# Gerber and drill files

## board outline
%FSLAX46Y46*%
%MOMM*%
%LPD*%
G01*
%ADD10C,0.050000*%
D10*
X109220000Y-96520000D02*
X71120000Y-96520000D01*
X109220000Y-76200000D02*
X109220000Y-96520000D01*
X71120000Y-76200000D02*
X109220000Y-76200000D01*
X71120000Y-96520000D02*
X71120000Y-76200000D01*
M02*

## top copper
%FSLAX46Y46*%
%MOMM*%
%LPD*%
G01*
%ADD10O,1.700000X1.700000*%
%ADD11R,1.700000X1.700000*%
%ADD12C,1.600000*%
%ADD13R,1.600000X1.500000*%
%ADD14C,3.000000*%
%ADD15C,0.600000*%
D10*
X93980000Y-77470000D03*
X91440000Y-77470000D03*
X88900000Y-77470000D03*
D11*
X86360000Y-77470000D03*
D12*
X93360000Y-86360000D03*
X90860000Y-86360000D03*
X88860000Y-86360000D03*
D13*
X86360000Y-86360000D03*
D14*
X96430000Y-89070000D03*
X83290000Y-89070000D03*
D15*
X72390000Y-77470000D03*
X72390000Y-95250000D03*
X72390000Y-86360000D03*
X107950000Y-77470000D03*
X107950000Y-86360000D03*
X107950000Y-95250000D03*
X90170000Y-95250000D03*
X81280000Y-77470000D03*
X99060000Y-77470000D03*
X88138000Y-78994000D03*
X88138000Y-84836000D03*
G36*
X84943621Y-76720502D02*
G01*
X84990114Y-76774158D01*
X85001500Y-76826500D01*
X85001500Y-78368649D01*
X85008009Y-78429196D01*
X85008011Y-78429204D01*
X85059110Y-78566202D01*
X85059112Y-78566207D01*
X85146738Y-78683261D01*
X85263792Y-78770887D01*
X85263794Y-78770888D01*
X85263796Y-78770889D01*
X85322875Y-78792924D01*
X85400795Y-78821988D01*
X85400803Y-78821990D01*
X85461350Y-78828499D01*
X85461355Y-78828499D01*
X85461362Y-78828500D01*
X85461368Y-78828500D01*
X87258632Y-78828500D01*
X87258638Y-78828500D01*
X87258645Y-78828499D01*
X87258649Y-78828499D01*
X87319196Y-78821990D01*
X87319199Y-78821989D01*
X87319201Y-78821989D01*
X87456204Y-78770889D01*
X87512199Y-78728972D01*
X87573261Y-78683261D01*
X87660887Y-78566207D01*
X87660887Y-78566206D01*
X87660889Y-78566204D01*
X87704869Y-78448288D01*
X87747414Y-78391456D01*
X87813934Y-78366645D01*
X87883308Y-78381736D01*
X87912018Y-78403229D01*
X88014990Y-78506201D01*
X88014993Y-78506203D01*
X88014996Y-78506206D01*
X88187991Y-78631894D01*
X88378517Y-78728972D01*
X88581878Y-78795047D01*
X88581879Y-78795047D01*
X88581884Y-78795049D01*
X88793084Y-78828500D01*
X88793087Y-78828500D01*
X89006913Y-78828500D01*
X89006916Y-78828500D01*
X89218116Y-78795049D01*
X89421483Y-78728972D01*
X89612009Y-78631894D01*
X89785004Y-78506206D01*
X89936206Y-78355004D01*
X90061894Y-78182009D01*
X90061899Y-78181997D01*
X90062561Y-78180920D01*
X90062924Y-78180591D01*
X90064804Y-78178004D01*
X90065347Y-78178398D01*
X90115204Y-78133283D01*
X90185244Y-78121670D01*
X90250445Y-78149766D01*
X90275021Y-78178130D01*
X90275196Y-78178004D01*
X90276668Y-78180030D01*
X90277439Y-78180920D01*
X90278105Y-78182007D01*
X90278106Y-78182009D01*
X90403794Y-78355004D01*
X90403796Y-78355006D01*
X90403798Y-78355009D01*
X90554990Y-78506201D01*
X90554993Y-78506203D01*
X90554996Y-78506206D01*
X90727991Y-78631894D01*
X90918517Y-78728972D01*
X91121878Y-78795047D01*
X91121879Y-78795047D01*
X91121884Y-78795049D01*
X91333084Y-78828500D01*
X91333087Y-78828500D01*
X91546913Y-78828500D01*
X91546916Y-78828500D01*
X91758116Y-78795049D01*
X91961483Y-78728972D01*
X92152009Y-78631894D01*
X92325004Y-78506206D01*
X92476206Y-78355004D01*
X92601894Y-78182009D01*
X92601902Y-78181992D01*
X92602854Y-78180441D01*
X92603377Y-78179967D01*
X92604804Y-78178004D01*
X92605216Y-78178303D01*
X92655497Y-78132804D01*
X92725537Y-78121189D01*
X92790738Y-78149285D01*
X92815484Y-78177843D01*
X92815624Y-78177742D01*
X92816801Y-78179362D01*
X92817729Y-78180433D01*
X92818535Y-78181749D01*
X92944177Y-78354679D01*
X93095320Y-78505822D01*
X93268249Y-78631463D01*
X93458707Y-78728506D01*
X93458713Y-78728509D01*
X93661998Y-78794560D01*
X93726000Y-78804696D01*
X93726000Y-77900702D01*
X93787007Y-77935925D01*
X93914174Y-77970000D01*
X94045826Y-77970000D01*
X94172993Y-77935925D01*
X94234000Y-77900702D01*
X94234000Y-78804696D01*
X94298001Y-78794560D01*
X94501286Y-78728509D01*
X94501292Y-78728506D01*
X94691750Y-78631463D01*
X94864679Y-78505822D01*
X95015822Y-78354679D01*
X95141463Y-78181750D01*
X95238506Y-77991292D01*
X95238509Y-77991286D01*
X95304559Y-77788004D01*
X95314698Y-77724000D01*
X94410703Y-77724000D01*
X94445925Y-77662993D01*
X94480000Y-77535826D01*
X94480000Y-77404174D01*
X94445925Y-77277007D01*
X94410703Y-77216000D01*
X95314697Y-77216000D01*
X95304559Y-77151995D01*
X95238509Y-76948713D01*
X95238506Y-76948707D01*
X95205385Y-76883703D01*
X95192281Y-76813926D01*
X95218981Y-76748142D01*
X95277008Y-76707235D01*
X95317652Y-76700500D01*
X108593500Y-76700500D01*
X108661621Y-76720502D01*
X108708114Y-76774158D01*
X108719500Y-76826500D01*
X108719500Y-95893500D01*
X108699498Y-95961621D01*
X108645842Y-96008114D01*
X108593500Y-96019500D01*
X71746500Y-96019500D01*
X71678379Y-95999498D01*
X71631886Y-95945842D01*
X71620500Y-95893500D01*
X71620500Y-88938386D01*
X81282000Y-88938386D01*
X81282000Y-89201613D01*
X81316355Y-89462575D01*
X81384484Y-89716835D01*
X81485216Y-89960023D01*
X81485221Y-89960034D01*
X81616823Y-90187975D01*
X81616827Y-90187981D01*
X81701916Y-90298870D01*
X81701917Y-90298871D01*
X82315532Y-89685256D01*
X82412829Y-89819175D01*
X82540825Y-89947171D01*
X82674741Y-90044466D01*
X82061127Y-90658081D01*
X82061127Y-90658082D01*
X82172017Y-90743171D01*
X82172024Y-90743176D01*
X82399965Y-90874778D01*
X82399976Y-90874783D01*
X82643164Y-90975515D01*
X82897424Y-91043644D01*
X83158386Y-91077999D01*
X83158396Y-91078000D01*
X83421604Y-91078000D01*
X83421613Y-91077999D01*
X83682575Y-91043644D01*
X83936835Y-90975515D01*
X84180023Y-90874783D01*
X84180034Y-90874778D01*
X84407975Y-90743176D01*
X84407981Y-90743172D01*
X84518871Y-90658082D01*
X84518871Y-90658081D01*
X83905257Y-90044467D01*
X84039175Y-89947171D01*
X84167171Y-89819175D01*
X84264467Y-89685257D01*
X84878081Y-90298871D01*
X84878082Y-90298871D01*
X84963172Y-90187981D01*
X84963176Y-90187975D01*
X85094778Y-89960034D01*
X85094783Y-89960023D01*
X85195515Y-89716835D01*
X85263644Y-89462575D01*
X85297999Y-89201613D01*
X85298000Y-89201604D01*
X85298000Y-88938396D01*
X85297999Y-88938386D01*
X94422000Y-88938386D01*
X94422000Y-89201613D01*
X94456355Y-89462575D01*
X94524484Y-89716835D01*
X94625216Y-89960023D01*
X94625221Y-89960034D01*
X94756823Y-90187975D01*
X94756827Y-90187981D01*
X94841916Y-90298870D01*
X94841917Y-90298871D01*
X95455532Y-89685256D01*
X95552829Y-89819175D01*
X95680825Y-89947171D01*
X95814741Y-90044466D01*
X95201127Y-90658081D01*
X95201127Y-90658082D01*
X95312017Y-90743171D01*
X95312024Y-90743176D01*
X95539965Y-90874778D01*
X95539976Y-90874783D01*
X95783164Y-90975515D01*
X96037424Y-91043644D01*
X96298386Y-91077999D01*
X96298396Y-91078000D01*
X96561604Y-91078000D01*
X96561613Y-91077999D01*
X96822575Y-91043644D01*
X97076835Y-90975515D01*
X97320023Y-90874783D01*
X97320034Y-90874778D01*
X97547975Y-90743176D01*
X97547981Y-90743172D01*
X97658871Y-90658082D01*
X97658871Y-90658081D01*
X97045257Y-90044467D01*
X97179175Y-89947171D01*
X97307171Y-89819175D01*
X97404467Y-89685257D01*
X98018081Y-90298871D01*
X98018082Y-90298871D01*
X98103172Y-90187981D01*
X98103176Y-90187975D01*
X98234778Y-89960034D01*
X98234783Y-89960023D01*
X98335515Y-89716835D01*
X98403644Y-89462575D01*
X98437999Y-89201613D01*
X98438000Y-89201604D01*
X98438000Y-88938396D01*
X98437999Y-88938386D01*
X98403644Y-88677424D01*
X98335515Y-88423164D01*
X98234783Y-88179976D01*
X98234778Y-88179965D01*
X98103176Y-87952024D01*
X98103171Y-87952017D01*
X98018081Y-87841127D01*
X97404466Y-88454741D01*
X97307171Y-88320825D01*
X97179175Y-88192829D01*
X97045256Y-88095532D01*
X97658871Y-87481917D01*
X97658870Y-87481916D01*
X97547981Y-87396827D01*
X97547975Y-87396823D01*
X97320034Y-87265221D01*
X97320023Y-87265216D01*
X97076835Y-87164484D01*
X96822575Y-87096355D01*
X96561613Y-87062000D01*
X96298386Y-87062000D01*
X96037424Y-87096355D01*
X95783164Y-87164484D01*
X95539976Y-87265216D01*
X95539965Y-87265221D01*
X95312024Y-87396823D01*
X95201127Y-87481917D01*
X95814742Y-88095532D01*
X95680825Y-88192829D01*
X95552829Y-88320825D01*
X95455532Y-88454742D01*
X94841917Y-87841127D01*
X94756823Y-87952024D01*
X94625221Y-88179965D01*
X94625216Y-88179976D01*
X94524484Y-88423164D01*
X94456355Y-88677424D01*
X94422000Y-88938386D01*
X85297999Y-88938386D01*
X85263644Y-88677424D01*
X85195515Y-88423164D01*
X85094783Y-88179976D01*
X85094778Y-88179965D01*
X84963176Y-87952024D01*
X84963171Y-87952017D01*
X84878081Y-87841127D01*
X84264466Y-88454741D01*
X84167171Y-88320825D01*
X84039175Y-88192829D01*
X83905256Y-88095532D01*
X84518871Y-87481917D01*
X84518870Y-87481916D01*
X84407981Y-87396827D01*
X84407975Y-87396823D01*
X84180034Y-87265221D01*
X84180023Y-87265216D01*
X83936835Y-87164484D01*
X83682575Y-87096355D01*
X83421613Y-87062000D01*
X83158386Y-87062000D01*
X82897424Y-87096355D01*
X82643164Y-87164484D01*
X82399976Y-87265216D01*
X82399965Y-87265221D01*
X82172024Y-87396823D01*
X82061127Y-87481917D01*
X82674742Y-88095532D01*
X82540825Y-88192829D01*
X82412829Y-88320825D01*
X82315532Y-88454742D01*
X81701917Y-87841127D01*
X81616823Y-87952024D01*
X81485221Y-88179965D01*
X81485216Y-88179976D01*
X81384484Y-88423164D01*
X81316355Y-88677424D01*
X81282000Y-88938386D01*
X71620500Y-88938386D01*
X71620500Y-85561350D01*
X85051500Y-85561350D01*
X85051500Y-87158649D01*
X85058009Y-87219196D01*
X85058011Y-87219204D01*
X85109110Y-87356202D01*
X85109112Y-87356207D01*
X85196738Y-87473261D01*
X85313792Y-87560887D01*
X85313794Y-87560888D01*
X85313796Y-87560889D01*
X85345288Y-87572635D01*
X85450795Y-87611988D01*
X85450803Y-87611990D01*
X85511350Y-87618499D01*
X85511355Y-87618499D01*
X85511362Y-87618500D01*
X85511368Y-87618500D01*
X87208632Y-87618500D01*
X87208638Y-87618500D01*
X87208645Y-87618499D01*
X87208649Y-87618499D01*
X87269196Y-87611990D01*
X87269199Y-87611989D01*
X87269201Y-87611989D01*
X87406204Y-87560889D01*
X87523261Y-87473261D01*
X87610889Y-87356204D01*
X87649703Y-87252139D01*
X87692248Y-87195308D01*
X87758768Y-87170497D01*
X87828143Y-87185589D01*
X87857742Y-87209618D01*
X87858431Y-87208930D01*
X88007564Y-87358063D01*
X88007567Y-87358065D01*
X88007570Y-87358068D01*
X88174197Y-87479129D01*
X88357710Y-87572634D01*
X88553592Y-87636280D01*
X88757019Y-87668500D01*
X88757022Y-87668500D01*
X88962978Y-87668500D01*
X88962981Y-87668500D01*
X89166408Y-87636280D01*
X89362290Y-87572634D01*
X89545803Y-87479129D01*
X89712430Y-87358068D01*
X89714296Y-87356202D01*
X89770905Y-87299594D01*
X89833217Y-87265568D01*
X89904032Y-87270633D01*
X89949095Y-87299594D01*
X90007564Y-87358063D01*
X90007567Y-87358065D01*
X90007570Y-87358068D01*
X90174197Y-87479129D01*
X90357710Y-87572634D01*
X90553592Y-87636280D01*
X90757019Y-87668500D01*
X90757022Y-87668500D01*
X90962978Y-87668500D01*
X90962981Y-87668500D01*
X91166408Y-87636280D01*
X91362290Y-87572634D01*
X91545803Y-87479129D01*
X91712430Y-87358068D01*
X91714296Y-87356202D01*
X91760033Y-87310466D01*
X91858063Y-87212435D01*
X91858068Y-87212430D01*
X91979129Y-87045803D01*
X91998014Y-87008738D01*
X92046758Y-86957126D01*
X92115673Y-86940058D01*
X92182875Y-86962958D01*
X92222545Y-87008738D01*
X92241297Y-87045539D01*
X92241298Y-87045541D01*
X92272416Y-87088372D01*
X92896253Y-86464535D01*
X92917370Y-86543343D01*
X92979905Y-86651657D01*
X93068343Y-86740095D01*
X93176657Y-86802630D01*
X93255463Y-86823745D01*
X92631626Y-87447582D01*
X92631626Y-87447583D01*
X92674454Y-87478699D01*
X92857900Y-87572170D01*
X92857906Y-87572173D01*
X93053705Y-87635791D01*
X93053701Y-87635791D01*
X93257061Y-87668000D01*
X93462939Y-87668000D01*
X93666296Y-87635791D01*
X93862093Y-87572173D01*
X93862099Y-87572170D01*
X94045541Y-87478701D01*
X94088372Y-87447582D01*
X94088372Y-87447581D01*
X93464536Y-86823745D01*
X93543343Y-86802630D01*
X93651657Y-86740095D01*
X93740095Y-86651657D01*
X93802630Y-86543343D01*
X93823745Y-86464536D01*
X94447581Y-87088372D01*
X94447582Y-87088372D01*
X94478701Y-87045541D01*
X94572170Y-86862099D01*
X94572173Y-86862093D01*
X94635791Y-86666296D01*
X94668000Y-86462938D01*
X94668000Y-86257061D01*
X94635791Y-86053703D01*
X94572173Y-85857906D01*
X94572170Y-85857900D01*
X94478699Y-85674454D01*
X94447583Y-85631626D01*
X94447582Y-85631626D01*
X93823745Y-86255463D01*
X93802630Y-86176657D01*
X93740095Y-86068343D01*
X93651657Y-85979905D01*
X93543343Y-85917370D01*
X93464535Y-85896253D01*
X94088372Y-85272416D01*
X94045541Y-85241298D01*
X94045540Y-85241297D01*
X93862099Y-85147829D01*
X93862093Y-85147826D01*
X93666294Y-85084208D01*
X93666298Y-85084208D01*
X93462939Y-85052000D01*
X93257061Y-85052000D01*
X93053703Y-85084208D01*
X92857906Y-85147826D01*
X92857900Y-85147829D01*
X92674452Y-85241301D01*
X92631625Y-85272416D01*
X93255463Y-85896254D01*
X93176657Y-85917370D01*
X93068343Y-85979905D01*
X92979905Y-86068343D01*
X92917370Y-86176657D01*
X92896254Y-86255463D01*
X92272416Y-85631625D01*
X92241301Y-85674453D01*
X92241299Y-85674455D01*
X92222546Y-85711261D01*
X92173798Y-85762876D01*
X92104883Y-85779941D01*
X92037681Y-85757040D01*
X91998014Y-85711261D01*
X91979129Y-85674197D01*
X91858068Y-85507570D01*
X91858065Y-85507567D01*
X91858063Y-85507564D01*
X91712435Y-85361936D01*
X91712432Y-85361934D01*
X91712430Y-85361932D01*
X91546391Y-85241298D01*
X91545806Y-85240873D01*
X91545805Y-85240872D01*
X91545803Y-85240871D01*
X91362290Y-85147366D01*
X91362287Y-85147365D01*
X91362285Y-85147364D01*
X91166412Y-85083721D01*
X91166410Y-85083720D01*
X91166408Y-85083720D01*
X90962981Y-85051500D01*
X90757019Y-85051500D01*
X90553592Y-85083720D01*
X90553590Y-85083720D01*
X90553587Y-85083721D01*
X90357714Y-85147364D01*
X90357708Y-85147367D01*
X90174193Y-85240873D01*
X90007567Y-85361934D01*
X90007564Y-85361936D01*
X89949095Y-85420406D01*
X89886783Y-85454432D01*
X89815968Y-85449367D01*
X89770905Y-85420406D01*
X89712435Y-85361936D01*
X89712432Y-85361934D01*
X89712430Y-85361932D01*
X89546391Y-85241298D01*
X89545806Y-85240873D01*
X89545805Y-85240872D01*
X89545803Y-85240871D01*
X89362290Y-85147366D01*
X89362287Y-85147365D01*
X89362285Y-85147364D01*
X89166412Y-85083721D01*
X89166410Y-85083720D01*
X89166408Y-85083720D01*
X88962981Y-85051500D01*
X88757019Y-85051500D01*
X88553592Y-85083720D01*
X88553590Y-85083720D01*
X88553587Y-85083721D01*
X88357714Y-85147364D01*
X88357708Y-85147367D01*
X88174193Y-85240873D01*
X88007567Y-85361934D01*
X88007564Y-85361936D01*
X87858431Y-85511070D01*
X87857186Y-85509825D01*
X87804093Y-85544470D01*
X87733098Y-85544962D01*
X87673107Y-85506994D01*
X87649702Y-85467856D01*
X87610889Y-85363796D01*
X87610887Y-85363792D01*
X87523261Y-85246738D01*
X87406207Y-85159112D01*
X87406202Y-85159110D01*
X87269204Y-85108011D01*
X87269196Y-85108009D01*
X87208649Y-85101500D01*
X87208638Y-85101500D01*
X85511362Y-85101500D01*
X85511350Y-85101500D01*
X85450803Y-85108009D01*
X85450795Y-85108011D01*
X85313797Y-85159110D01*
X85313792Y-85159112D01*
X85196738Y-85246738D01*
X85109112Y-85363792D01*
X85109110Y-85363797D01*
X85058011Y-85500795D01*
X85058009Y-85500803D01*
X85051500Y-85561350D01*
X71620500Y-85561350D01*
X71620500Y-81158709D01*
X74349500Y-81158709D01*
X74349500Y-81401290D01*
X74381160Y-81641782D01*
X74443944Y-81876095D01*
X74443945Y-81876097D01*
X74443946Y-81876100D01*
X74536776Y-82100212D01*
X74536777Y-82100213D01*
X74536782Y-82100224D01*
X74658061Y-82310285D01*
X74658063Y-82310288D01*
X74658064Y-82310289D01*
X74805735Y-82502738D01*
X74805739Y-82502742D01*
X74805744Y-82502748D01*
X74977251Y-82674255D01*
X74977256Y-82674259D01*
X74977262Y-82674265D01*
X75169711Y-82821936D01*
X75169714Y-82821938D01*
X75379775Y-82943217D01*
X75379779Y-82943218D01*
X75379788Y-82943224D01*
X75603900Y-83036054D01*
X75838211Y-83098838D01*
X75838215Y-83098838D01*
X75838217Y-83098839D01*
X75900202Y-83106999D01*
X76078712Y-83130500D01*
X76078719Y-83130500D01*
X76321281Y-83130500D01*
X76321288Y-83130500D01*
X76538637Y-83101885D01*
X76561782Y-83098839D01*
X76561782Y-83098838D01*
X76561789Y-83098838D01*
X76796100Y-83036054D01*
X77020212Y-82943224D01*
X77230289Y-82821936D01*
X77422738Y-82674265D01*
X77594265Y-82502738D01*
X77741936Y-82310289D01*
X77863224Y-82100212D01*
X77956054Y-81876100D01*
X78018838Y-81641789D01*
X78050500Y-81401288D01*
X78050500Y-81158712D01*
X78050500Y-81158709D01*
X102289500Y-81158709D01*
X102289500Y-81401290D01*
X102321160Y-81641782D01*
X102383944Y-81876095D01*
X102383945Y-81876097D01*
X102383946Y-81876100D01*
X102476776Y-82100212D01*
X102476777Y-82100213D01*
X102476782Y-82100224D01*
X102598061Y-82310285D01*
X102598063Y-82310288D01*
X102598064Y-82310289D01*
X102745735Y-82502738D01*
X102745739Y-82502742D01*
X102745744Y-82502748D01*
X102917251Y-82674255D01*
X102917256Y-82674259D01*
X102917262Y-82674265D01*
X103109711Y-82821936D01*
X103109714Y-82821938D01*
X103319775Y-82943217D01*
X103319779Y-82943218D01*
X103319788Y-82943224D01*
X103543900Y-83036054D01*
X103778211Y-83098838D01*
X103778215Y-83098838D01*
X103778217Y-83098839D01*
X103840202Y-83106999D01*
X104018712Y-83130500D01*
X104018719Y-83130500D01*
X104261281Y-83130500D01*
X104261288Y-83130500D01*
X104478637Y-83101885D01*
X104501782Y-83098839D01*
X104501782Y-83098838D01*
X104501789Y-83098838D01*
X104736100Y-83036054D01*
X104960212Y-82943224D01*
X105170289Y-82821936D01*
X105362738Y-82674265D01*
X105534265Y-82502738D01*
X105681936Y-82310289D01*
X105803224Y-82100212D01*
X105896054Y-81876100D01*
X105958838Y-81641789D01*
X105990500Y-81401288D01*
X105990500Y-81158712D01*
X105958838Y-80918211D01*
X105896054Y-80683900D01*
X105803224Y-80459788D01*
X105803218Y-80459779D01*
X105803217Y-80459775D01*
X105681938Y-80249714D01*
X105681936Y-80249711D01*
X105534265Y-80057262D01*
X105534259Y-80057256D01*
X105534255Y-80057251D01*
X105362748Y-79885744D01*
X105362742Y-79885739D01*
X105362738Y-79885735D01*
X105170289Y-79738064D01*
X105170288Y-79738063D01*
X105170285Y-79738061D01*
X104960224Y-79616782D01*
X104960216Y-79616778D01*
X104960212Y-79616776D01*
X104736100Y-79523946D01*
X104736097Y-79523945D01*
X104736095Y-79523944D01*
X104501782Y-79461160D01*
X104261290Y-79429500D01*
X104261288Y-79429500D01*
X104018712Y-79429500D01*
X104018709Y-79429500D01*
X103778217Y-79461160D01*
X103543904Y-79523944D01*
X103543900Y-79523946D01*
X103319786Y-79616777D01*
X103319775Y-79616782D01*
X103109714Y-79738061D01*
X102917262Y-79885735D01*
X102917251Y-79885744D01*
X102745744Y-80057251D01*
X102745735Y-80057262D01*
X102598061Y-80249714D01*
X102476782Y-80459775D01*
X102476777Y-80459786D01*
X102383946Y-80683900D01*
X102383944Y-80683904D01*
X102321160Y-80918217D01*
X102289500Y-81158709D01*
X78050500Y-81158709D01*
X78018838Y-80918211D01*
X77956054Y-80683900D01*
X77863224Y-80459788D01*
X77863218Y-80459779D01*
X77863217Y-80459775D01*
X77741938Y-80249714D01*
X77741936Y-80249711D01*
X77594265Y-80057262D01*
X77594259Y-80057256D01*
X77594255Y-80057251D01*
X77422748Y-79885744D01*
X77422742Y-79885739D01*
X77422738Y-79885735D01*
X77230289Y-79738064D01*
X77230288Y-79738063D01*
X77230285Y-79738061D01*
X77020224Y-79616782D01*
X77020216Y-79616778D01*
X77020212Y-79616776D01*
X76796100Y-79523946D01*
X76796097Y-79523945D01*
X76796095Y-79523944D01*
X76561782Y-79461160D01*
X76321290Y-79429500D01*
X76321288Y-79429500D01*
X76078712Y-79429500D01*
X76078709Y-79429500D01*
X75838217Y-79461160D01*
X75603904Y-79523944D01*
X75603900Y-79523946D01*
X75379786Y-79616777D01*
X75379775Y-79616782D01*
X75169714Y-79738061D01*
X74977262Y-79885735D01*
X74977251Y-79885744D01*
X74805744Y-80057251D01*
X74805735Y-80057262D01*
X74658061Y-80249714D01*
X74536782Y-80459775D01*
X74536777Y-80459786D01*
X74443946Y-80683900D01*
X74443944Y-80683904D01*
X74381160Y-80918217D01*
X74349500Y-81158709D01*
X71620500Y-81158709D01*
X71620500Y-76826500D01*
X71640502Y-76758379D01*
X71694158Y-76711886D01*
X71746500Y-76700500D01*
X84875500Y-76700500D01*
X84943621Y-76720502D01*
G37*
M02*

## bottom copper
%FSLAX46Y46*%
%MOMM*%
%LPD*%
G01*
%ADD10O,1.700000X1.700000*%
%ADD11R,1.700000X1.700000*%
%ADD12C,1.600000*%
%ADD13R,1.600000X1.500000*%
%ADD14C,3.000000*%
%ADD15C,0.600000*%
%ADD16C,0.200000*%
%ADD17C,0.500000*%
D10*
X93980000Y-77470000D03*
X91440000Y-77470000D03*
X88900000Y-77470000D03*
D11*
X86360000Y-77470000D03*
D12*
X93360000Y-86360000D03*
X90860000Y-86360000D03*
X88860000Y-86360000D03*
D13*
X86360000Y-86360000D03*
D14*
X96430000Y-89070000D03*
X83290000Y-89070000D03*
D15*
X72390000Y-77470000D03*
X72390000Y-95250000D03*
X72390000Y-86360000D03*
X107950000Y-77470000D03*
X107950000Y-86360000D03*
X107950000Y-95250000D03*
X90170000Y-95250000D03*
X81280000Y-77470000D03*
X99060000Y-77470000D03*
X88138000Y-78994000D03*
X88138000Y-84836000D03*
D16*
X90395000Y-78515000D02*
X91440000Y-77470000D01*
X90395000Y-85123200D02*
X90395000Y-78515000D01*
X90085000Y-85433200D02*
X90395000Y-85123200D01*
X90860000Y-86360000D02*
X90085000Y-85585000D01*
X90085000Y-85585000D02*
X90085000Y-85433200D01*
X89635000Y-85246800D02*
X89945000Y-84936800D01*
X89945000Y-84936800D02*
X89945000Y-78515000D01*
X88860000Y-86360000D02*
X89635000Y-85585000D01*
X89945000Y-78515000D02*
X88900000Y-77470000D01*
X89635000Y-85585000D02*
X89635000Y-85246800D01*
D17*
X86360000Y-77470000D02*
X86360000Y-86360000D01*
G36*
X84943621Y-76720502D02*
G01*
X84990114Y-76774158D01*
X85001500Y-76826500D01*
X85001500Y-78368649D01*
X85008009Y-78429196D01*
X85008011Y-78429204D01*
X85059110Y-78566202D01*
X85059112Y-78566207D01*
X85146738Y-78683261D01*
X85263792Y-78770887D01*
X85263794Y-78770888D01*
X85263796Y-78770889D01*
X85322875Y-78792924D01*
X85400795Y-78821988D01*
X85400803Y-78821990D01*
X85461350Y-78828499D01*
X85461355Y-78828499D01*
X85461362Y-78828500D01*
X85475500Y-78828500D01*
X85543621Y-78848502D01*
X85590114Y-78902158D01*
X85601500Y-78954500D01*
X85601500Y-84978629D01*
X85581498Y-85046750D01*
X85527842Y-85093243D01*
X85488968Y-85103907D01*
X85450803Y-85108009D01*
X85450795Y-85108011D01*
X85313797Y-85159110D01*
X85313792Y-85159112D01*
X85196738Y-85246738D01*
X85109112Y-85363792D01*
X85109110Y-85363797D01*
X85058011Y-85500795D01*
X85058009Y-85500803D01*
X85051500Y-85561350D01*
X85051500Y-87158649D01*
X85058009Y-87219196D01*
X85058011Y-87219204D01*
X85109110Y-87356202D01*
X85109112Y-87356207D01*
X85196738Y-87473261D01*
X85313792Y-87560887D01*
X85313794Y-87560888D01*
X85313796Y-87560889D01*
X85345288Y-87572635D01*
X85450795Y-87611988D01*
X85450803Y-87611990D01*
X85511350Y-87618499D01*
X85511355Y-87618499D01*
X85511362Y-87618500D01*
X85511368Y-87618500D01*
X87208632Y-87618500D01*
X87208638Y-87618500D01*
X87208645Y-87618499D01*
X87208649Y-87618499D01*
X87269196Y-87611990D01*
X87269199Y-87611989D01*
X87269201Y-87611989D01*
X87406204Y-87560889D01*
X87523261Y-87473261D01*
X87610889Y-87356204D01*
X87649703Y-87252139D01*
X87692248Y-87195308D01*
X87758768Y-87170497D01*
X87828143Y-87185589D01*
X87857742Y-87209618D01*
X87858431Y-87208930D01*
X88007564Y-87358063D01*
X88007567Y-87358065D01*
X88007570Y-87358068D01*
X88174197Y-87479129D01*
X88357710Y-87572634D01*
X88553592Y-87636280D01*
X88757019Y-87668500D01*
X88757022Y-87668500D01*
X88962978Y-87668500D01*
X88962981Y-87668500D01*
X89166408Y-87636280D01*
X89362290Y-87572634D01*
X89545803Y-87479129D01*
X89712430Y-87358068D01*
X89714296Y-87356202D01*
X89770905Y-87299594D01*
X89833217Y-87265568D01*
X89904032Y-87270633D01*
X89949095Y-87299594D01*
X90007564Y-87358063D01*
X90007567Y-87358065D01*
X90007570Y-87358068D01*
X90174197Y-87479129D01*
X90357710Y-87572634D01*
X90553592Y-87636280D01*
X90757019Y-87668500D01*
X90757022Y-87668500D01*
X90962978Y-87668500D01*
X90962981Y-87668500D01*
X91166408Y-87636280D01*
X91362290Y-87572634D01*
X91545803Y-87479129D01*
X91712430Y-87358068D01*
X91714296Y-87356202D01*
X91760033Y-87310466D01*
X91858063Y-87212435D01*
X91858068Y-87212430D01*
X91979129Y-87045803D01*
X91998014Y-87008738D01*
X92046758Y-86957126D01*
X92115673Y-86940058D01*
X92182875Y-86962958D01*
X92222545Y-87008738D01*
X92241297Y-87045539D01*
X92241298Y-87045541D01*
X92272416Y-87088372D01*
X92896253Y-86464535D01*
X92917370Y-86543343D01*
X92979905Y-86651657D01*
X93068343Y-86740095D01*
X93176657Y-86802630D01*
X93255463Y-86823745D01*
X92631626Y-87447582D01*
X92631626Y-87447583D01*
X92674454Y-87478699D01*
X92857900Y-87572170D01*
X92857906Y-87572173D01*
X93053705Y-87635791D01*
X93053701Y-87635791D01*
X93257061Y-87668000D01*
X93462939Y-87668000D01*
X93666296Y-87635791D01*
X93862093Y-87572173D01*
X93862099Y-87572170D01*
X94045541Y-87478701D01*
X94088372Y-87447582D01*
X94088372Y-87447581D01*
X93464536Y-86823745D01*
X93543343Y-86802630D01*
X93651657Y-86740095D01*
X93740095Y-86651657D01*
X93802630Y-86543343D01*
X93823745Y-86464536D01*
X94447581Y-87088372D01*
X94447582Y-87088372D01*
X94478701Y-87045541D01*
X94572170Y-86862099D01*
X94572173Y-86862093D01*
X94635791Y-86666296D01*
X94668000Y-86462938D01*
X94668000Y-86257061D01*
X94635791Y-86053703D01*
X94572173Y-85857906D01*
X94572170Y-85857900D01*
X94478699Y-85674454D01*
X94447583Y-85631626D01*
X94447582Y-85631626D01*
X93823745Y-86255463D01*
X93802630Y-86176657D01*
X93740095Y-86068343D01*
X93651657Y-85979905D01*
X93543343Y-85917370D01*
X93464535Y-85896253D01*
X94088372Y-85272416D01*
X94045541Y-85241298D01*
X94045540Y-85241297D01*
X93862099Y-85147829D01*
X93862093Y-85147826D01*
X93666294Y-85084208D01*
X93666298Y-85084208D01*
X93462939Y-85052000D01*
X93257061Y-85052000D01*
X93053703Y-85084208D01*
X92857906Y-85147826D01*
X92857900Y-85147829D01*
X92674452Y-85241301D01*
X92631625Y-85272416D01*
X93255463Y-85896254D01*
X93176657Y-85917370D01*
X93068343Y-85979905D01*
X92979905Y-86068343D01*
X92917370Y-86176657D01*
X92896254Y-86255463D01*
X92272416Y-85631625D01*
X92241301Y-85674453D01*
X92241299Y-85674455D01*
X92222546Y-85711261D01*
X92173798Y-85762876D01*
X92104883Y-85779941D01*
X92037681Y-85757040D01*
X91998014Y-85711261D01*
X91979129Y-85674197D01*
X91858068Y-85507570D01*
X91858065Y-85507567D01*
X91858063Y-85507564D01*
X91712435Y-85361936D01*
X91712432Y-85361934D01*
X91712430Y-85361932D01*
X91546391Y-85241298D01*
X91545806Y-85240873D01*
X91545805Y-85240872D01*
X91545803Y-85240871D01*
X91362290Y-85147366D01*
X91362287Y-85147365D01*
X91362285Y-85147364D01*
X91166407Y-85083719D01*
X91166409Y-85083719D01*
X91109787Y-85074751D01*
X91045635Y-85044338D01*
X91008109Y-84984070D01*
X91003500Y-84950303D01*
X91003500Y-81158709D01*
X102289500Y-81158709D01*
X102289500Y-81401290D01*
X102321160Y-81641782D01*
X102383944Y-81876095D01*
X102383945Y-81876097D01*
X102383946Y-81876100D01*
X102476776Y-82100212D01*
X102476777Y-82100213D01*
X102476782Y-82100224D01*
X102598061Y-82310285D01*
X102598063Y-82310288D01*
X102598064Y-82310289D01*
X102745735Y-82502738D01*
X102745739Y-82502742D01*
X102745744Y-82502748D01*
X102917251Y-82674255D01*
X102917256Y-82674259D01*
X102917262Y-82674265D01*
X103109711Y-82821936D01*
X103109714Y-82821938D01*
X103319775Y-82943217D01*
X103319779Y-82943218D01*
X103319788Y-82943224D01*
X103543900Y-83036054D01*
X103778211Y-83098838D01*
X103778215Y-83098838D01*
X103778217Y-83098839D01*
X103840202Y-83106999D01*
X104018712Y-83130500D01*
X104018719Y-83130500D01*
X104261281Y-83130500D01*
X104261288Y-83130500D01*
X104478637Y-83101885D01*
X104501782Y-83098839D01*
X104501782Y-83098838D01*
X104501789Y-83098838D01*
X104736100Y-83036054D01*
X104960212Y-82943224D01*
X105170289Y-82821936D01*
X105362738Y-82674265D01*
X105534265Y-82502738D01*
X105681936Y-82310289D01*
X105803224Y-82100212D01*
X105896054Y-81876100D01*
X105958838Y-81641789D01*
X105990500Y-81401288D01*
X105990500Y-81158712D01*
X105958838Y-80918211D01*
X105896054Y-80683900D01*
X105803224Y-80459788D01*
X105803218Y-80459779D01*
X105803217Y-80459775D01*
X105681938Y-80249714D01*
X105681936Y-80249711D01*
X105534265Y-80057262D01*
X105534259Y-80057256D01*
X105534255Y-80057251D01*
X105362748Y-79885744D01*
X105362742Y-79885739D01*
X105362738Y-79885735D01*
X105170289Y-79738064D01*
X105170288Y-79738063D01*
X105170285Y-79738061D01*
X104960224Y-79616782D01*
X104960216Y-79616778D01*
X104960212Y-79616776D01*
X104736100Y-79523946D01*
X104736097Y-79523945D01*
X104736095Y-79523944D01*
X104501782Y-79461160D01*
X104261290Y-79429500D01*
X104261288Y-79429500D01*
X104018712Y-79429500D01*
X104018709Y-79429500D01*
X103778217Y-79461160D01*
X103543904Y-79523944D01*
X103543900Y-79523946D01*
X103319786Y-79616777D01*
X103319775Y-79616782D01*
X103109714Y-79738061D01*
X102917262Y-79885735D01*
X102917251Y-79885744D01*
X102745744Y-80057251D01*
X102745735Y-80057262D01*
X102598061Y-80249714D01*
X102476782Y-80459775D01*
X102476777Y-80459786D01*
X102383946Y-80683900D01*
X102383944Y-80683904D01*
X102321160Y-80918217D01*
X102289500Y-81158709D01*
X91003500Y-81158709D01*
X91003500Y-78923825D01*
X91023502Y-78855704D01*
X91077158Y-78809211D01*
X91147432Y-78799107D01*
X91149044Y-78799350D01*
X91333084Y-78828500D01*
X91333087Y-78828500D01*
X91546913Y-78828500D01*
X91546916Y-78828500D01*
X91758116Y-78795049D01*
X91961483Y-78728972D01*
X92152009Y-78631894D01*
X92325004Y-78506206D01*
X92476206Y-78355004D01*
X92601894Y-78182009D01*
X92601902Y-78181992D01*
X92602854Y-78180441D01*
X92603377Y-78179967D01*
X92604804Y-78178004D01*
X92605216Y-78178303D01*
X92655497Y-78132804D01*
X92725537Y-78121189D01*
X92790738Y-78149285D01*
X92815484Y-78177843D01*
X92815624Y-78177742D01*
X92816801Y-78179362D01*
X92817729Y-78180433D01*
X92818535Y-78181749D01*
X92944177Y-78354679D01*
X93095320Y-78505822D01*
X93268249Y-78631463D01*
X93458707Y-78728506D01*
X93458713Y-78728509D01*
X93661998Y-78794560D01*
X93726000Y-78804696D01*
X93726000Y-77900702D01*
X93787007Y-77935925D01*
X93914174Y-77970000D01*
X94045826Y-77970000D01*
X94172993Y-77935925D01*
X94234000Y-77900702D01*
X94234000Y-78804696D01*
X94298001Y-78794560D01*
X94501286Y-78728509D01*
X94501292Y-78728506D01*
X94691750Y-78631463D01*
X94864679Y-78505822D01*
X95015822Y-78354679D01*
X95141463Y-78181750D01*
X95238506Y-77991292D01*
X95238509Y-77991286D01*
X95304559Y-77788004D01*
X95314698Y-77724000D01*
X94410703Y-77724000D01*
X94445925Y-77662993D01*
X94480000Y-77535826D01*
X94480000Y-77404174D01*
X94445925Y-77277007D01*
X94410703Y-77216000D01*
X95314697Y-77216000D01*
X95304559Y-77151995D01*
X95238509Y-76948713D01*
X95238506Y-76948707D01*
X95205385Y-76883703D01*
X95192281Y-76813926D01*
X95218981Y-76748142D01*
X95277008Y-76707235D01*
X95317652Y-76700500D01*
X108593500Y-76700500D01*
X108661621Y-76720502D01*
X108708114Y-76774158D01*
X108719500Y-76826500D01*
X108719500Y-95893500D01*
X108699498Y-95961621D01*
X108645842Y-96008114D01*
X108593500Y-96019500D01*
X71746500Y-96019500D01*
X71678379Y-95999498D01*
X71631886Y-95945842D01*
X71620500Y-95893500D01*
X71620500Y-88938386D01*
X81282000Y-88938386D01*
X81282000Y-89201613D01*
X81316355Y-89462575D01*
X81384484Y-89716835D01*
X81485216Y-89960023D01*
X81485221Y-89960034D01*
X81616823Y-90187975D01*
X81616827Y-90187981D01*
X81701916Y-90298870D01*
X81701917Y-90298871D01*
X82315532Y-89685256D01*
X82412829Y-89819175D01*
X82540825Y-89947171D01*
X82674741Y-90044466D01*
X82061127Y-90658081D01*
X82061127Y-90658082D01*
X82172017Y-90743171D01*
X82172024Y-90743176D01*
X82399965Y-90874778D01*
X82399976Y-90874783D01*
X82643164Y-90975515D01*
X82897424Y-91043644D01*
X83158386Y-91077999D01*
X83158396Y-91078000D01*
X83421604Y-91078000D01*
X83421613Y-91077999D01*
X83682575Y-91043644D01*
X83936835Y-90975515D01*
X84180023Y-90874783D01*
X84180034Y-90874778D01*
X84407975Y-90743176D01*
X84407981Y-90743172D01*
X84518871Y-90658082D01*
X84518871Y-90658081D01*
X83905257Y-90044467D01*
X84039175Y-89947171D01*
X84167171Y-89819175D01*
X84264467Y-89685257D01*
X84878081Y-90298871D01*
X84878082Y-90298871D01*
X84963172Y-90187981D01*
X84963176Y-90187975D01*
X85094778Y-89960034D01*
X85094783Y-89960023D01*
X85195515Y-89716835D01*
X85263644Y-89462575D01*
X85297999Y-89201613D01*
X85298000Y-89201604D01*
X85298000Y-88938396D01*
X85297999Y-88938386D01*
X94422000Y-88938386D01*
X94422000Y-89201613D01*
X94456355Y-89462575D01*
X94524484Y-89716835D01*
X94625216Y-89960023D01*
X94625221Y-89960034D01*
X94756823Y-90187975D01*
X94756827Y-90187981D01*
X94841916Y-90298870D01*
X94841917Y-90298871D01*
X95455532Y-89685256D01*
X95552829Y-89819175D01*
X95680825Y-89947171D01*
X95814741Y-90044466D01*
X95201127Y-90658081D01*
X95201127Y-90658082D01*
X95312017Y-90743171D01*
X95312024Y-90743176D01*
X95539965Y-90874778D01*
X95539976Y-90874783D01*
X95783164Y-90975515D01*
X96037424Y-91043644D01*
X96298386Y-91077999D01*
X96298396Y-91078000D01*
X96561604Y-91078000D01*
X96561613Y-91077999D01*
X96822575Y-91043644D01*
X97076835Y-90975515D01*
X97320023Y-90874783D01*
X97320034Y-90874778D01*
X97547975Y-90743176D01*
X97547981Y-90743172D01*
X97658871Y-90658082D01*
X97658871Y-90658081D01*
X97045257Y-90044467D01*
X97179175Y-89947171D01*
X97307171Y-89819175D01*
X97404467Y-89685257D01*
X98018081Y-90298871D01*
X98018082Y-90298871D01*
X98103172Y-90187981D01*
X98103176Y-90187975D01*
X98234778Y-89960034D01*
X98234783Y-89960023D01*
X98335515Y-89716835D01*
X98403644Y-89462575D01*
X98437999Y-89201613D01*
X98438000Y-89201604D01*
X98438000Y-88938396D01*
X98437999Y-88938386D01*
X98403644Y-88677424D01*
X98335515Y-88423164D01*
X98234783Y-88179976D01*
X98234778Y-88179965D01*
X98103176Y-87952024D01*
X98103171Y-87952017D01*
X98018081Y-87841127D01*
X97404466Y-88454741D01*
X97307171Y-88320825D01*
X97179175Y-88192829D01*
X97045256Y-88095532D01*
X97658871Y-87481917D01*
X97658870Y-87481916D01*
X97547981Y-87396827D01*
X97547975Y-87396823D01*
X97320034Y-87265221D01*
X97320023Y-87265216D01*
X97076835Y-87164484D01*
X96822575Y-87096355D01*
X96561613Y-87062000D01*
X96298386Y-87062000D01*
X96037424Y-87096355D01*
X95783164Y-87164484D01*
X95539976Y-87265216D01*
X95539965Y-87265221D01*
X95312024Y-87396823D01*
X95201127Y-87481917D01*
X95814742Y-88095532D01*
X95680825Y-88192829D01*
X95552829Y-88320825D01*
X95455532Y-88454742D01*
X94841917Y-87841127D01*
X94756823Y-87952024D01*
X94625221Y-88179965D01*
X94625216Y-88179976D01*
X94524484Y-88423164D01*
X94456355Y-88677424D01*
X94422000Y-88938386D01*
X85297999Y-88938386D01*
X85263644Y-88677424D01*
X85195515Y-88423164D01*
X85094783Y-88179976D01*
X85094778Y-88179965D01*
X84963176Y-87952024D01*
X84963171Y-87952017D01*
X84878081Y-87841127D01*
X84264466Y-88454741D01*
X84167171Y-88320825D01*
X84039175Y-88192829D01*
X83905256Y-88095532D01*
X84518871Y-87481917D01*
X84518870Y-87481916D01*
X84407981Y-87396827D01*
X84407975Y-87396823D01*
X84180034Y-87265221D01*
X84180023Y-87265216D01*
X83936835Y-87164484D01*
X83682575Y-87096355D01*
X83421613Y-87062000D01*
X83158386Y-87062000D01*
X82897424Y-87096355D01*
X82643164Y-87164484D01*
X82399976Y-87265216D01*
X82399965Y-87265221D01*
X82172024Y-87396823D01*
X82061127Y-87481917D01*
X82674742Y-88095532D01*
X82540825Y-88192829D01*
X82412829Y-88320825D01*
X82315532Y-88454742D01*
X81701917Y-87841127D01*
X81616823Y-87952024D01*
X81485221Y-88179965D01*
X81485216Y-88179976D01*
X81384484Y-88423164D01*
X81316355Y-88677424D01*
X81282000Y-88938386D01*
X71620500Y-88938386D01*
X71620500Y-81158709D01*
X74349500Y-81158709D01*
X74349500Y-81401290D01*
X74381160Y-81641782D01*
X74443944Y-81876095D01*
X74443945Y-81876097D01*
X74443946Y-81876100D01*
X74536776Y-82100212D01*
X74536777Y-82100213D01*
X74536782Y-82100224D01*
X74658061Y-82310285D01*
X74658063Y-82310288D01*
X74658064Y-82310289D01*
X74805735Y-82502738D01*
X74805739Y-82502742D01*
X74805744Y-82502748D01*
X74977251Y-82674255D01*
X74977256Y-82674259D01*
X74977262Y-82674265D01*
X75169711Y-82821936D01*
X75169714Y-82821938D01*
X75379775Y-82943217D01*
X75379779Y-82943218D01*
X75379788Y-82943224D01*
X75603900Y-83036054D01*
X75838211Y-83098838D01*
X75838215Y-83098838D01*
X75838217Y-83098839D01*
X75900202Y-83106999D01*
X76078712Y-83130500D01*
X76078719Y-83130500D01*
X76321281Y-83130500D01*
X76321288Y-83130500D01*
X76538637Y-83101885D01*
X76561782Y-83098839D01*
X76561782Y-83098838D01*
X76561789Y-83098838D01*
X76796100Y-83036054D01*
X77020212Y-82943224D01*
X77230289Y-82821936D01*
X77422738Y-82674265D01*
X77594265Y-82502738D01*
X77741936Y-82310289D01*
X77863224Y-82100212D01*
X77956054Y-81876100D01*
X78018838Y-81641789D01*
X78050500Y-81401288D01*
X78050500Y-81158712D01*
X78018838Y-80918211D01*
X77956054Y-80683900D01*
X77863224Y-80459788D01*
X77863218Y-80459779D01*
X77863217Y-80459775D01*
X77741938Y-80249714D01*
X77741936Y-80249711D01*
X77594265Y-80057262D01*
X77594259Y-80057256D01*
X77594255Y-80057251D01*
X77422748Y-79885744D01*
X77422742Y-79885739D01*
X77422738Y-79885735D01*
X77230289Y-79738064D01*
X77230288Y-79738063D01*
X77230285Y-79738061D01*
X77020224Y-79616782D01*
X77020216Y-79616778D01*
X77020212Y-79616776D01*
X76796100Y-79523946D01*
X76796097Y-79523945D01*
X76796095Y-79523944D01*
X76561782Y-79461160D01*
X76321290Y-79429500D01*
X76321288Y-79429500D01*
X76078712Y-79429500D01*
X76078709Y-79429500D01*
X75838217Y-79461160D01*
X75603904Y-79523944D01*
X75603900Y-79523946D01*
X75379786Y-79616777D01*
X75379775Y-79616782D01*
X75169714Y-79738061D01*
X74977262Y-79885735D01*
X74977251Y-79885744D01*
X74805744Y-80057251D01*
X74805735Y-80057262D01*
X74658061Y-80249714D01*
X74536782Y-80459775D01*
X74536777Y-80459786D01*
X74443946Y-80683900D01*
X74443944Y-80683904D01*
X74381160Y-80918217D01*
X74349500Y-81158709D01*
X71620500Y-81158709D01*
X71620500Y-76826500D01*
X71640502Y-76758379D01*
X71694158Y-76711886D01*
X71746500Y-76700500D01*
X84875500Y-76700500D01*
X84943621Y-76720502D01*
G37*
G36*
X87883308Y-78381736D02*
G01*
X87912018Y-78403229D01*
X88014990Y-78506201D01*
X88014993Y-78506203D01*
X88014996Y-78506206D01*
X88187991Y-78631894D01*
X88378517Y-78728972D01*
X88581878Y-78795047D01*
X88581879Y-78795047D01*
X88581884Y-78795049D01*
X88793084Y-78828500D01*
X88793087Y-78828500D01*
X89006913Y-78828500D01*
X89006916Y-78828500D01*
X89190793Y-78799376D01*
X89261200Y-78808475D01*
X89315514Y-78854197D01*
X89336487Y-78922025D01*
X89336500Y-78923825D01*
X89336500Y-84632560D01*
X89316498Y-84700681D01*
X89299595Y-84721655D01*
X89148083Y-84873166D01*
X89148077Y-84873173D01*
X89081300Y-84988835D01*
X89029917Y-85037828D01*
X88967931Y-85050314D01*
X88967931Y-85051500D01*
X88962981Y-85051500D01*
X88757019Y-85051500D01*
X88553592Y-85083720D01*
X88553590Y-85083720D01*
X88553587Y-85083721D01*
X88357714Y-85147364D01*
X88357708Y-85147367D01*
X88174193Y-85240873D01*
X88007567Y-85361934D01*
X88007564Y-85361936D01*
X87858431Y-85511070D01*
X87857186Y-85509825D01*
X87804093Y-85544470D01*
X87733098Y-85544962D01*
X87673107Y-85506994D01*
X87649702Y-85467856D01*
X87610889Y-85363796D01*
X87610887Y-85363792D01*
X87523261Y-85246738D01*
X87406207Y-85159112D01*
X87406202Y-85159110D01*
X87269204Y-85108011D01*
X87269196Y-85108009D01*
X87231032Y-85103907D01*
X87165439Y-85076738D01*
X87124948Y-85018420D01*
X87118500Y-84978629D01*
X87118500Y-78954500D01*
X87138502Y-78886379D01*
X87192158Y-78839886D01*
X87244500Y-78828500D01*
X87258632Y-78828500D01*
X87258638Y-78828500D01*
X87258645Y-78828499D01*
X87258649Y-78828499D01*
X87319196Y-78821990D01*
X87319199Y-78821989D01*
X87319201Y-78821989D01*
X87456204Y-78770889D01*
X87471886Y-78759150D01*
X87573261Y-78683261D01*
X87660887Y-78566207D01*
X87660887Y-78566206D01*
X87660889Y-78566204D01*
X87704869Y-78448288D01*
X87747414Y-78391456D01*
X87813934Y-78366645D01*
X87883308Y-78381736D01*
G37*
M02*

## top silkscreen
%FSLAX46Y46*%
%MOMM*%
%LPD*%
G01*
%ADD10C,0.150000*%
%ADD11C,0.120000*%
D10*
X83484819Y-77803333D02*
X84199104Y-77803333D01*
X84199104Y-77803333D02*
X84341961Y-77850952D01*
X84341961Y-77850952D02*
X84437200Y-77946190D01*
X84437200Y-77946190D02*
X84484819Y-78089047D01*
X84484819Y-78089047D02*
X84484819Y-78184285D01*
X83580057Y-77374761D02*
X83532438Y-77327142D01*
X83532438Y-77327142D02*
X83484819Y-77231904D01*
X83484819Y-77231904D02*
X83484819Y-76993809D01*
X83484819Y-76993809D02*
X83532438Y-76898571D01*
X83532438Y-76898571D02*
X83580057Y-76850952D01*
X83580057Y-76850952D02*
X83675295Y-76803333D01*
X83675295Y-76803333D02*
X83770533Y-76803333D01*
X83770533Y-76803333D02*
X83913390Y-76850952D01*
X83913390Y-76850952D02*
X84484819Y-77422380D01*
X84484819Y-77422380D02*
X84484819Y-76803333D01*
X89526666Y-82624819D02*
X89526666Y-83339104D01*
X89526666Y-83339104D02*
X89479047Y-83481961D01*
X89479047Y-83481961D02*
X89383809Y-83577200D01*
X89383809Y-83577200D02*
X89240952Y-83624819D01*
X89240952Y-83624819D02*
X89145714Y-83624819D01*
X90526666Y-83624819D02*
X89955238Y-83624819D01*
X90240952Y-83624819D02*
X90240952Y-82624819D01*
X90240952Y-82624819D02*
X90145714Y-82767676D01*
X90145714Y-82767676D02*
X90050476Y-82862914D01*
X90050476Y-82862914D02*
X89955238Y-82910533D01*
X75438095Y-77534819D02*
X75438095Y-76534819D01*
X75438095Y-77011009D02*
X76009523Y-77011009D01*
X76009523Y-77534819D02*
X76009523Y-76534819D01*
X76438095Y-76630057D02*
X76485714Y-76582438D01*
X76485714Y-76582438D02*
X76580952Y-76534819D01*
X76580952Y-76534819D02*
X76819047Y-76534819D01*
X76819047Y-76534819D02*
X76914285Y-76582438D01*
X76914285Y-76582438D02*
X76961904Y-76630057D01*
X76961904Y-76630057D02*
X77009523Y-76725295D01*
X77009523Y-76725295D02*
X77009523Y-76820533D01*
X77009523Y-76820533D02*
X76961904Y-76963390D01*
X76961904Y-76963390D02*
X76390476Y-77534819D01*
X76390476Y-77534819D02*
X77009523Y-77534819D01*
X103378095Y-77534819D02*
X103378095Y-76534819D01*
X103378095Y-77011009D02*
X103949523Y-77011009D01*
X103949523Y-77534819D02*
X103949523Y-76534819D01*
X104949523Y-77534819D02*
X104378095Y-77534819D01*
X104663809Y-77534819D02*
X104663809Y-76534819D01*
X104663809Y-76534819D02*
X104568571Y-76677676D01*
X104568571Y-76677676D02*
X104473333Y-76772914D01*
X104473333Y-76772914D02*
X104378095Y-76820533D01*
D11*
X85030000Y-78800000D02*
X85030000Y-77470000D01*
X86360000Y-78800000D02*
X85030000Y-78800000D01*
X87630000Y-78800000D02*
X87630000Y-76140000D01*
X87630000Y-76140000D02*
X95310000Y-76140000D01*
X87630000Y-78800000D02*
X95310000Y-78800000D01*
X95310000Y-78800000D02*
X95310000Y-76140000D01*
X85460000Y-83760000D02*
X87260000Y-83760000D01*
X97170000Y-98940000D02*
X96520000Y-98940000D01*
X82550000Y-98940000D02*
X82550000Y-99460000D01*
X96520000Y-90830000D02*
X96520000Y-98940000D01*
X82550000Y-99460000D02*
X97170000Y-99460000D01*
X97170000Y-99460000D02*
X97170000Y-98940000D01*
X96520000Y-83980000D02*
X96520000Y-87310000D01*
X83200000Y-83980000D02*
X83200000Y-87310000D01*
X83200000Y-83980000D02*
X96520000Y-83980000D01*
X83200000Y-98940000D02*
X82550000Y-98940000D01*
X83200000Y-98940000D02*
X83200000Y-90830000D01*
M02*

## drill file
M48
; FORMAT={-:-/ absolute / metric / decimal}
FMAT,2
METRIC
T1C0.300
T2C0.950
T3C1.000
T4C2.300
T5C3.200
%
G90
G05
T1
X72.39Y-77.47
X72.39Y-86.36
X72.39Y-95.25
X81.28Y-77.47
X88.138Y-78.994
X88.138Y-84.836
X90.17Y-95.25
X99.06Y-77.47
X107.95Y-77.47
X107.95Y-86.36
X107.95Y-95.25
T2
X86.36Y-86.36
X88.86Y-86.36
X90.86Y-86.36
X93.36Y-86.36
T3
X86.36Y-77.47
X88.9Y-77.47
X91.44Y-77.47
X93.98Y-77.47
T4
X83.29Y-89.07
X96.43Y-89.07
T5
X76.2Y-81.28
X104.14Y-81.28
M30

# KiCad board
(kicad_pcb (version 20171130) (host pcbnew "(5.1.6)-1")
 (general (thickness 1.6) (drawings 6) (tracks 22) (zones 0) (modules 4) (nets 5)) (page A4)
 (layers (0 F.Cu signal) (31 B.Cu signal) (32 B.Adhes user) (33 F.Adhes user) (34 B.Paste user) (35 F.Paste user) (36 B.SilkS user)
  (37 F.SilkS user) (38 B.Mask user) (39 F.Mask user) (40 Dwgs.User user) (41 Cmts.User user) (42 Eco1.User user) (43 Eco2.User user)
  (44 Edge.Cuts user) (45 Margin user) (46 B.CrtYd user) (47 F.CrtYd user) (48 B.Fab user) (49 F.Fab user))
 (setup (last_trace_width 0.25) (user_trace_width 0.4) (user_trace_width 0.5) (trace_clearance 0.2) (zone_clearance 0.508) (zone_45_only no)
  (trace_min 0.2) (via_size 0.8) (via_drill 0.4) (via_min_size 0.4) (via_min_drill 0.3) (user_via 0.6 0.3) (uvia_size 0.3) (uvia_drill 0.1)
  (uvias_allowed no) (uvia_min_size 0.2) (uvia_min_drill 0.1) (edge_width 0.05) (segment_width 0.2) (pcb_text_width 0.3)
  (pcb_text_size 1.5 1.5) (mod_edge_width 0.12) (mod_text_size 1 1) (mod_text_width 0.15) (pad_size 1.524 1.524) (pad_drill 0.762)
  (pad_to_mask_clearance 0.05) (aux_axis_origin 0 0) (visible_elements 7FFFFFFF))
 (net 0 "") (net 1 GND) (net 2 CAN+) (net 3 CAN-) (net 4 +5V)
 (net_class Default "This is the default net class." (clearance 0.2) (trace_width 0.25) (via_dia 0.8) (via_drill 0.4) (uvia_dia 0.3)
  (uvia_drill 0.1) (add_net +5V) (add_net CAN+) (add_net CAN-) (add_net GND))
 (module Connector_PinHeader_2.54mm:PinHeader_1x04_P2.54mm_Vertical (layer F.Cu) (at 86.36 77.47 90)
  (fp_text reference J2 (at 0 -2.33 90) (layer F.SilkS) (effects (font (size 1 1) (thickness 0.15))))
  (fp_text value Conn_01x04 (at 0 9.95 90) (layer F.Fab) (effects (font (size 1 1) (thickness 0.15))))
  (fp_line (start -1.33 -1.33) (end 0 -1.33) (layer F.SilkS) (width 0.12))
  (fp_line (start -1.33 0) (end -1.33 -1.33) (layer F.SilkS) (width 0.12))
  (fp_line (start -1.33 1.27) (end 1.33 1.27) (layer F.SilkS) (width 0.12))
  (fp_line (start 1.33 1.27) (end 1.33 8.95) (layer F.SilkS) (width 0.12))
  (fp_line (start -1.33 1.27) (end -1.33 8.95) (layer F.SilkS) (width 0.12))
  (fp_line (start -1.33 8.95) (end 1.33 8.95) (layer F.SilkS) (width 0.12))
  (pad 4 thru_hole oval (at 0 7.62 90) (size 1.7 1.7) (drill 1) (layers *.Cu *.Mask) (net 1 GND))
  (pad 3 thru_hole oval (at 0 5.08 90) (size 1.7 1.7) (drill 1) (layers *.Cu *.Mask) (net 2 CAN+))
  (pad 2 thru_hole oval (at 0 2.54 90) (size 1.7 1.7) (drill 1) (layers *.Cu *.Mask) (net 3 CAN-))
  (pad 1 thru_hole rect (at 0 0 90) (size 1.7 1.7) (drill 1) (layers *.Cu *.Mask) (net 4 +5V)))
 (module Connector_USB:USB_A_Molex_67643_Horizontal (layer F.Cu) (at 86.36 86.36)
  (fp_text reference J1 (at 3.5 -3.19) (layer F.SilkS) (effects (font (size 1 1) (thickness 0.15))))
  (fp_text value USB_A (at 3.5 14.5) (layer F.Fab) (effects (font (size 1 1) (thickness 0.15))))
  (fp_line (start -0.9 -2.6) (end 0.9 -2.6) (layer F.SilkS) (width 0.12))
  (fp_line (start 10.81 12.58) (end 10.16 12.58) (layer F.SilkS) (width 0.12))
  (fp_line (start -3.81 12.58) (end -3.81 13.1) (layer F.SilkS) (width 0.12))
  (fp_line (start 10.16 4.47) (end 10.16 12.58) (layer F.SilkS) (width 0.12))
  (fp_line (start -3.81 13.1) (end 10.81 13.1) (layer F.SilkS) (width 0.12))
  (fp_line (start 10.81 13.1) (end 10.81 12.58) (layer F.SilkS) (width 0.12))
  (fp_line (start 10.16 -2.38) (end 10.16 0.95) (layer F.SilkS) (width 0.12))
  (fp_line (start -3.16 -2.38) (end -3.16 0.95) (layer F.SilkS) (width 0.12))
  (fp_line (start -3.16 -2.38) (end 10.16 -2.38) (layer F.SilkS) (width 0.12))
  (fp_line (start -3.16 12.58) (end -3.81 12.58) (layer F.SilkS) (width 0.12))
  (fp_line (start -3.16 12.58) (end -3.16 4.47) (layer F.SilkS) (width 0.12))
  (pad 4 thru_hole circle (at 7 0) (size 1.6 1.6) (drill 0.95) (layers *.Cu *.Mask) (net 1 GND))
  (pad 3 thru_hole circle (at 4.5 0) (size 1.6 1.6) (drill 0.95) (layers *.Cu *.Mask) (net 2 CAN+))
  (pad 2 thru_hole circle (at 2.5 0) (size 1.6 1.6) (drill 0.95) (layers *.Cu *.Mask) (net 3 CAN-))
  (pad 1 thru_hole rect (at 0 0) (size 1.6 1.5) (drill 0.95) (layers *.Cu *.Mask) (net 4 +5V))
  (pad 5 thru_hole circle (at 10.07 2.71) (size 3 3) (drill 2.3) (layers *.Cu *.Mask) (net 1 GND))
  (pad 5 thru_hole circle (at -3.07 2.71) (size 3 3) (drill 2.3) (layers *.Cu *.Mask) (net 1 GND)))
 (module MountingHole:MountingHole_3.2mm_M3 (layer F.Cu) (at 76.2 81.28)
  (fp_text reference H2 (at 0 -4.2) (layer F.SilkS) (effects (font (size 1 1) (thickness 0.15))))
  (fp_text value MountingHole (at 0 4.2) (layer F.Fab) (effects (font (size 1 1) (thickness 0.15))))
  (pad 1 np_thru_hole circle (at 0 0) (size 3.2 3.2) (drill 3.2) (layers *.Cu *.Mask)))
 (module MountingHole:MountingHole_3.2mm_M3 (layer F.Cu) (at 104.14 81.28)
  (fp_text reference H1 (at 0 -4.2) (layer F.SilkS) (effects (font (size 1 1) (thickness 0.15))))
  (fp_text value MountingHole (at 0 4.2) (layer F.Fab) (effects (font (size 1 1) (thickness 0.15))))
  (pad 1 np_thru_hole circle (at 0 0) (size 3.2 3.2) (drill 3.2) (layers *.Cu *.Mask)))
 (gr_line (start 109.22 96.52) (end 71.12 96.52) (layer Edge.Cuts) (width 0.05))
 (gr_line (start 109.22 76.2) (end 109.22 96.52) (layer Edge.Cuts) (width 0.05))
 (gr_line (start 71.12 76.2) (end 109.22 76.2) (layer Edge.Cuts) (width 0.05))
 (gr_line (start 71.12 96.52) (end 71.12 76.2) (layer Edge.Cuts) (width 0.05))
 (via (at 72.39 77.47) (size 0.6) (drill 0.3) (layers F.Cu B.Cu) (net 1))
 (via (at 72.39 95.25) (size 0.6) (drill 0.3) (layers F.Cu B.Cu) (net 1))
 (via (at 72.39 86.36) (size 0.6) (drill 0.3) (layers F.Cu B.Cu) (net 1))
 (via (at 107.95 77.47) (size 0.6) (drill 0.3) (layers F.Cu B.Cu) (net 1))
 (via (at 107.95 86.36) (size 0.6) (drill 0.3) (layers F.Cu B.Cu) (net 1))
 (via (at 107.95 95.25) (size 0.6) (drill 0.3) (layers F.Cu B.Cu) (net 1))
 (via (at 90.17 95.25) (size 0.6) (drill 0.3) (layers F.Cu B.Cu) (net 1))
 (via (at 81.28 77.47) (size 0.6) (drill 0.3) (layers F.Cu B.Cu) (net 1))
 (via (at 99.06 77.47) (size 0.6) (drill 0.3) (layers F.Cu B.Cu) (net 1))
 (via (at 88.138 78.994) (size 0.6) (drill 0.3) (layers F.Cu B.Cu) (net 1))
 (via (at 88.138 84.836) (size 0.6) (drill 0.3) (layers F.Cu B.Cu) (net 1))
 (segment (start 90.395 78.515) (end 91.44 77.47) (width 0.2) (layer B.Cu) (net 2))
 (segment (start 90.395 85.1232) (end 90.395 78.515) (width 0.2) (layer B.Cu) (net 2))
 (segment (start 90.085 85.4332) (end 90.395 85.1232) (width 0.2) (layer B.Cu) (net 2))
 (segment (start 90.86 86.36) (end 90.085 85.585) (width 0.2) (layer B.Cu) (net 2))
 (segment (start 90.085 85.585) (end 90.085 85.4332) (width 0.2) (layer B.Cu) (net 2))
 (segment (start 89.635 85.2468) (end 89.945 84.9368) (width 0.2) (layer B.Cu) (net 3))
 (segment (start 89.945 84.9368) (end 89.945 78.515) (width 0.2) (layer B.Cu) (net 3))
 (segment (start 88.86 86.36) (end 89.635 85.585) (width 0.2) (layer B.Cu) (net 3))
 (segment (start 89.945 78.515) (end 88.9 77.47) (width 0.2) (layer B.Cu) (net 3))
 (segment (start 89.635 85.585) (end 89.635 85.2468) (width 0.2) (layer B.Cu) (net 3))
 (segment (start 86.36 77.47) (end 86.36 86.36) (width 0.5) (layer B.Cu) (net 4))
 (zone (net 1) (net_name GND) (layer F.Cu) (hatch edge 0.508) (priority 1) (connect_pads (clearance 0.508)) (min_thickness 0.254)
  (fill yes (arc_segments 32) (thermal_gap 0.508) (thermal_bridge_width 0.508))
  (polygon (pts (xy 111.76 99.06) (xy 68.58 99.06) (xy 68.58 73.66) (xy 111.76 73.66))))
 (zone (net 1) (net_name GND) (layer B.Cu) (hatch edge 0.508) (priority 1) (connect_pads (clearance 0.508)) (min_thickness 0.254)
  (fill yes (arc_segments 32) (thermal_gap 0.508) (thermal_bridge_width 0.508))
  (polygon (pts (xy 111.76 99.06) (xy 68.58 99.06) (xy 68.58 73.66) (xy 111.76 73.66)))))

